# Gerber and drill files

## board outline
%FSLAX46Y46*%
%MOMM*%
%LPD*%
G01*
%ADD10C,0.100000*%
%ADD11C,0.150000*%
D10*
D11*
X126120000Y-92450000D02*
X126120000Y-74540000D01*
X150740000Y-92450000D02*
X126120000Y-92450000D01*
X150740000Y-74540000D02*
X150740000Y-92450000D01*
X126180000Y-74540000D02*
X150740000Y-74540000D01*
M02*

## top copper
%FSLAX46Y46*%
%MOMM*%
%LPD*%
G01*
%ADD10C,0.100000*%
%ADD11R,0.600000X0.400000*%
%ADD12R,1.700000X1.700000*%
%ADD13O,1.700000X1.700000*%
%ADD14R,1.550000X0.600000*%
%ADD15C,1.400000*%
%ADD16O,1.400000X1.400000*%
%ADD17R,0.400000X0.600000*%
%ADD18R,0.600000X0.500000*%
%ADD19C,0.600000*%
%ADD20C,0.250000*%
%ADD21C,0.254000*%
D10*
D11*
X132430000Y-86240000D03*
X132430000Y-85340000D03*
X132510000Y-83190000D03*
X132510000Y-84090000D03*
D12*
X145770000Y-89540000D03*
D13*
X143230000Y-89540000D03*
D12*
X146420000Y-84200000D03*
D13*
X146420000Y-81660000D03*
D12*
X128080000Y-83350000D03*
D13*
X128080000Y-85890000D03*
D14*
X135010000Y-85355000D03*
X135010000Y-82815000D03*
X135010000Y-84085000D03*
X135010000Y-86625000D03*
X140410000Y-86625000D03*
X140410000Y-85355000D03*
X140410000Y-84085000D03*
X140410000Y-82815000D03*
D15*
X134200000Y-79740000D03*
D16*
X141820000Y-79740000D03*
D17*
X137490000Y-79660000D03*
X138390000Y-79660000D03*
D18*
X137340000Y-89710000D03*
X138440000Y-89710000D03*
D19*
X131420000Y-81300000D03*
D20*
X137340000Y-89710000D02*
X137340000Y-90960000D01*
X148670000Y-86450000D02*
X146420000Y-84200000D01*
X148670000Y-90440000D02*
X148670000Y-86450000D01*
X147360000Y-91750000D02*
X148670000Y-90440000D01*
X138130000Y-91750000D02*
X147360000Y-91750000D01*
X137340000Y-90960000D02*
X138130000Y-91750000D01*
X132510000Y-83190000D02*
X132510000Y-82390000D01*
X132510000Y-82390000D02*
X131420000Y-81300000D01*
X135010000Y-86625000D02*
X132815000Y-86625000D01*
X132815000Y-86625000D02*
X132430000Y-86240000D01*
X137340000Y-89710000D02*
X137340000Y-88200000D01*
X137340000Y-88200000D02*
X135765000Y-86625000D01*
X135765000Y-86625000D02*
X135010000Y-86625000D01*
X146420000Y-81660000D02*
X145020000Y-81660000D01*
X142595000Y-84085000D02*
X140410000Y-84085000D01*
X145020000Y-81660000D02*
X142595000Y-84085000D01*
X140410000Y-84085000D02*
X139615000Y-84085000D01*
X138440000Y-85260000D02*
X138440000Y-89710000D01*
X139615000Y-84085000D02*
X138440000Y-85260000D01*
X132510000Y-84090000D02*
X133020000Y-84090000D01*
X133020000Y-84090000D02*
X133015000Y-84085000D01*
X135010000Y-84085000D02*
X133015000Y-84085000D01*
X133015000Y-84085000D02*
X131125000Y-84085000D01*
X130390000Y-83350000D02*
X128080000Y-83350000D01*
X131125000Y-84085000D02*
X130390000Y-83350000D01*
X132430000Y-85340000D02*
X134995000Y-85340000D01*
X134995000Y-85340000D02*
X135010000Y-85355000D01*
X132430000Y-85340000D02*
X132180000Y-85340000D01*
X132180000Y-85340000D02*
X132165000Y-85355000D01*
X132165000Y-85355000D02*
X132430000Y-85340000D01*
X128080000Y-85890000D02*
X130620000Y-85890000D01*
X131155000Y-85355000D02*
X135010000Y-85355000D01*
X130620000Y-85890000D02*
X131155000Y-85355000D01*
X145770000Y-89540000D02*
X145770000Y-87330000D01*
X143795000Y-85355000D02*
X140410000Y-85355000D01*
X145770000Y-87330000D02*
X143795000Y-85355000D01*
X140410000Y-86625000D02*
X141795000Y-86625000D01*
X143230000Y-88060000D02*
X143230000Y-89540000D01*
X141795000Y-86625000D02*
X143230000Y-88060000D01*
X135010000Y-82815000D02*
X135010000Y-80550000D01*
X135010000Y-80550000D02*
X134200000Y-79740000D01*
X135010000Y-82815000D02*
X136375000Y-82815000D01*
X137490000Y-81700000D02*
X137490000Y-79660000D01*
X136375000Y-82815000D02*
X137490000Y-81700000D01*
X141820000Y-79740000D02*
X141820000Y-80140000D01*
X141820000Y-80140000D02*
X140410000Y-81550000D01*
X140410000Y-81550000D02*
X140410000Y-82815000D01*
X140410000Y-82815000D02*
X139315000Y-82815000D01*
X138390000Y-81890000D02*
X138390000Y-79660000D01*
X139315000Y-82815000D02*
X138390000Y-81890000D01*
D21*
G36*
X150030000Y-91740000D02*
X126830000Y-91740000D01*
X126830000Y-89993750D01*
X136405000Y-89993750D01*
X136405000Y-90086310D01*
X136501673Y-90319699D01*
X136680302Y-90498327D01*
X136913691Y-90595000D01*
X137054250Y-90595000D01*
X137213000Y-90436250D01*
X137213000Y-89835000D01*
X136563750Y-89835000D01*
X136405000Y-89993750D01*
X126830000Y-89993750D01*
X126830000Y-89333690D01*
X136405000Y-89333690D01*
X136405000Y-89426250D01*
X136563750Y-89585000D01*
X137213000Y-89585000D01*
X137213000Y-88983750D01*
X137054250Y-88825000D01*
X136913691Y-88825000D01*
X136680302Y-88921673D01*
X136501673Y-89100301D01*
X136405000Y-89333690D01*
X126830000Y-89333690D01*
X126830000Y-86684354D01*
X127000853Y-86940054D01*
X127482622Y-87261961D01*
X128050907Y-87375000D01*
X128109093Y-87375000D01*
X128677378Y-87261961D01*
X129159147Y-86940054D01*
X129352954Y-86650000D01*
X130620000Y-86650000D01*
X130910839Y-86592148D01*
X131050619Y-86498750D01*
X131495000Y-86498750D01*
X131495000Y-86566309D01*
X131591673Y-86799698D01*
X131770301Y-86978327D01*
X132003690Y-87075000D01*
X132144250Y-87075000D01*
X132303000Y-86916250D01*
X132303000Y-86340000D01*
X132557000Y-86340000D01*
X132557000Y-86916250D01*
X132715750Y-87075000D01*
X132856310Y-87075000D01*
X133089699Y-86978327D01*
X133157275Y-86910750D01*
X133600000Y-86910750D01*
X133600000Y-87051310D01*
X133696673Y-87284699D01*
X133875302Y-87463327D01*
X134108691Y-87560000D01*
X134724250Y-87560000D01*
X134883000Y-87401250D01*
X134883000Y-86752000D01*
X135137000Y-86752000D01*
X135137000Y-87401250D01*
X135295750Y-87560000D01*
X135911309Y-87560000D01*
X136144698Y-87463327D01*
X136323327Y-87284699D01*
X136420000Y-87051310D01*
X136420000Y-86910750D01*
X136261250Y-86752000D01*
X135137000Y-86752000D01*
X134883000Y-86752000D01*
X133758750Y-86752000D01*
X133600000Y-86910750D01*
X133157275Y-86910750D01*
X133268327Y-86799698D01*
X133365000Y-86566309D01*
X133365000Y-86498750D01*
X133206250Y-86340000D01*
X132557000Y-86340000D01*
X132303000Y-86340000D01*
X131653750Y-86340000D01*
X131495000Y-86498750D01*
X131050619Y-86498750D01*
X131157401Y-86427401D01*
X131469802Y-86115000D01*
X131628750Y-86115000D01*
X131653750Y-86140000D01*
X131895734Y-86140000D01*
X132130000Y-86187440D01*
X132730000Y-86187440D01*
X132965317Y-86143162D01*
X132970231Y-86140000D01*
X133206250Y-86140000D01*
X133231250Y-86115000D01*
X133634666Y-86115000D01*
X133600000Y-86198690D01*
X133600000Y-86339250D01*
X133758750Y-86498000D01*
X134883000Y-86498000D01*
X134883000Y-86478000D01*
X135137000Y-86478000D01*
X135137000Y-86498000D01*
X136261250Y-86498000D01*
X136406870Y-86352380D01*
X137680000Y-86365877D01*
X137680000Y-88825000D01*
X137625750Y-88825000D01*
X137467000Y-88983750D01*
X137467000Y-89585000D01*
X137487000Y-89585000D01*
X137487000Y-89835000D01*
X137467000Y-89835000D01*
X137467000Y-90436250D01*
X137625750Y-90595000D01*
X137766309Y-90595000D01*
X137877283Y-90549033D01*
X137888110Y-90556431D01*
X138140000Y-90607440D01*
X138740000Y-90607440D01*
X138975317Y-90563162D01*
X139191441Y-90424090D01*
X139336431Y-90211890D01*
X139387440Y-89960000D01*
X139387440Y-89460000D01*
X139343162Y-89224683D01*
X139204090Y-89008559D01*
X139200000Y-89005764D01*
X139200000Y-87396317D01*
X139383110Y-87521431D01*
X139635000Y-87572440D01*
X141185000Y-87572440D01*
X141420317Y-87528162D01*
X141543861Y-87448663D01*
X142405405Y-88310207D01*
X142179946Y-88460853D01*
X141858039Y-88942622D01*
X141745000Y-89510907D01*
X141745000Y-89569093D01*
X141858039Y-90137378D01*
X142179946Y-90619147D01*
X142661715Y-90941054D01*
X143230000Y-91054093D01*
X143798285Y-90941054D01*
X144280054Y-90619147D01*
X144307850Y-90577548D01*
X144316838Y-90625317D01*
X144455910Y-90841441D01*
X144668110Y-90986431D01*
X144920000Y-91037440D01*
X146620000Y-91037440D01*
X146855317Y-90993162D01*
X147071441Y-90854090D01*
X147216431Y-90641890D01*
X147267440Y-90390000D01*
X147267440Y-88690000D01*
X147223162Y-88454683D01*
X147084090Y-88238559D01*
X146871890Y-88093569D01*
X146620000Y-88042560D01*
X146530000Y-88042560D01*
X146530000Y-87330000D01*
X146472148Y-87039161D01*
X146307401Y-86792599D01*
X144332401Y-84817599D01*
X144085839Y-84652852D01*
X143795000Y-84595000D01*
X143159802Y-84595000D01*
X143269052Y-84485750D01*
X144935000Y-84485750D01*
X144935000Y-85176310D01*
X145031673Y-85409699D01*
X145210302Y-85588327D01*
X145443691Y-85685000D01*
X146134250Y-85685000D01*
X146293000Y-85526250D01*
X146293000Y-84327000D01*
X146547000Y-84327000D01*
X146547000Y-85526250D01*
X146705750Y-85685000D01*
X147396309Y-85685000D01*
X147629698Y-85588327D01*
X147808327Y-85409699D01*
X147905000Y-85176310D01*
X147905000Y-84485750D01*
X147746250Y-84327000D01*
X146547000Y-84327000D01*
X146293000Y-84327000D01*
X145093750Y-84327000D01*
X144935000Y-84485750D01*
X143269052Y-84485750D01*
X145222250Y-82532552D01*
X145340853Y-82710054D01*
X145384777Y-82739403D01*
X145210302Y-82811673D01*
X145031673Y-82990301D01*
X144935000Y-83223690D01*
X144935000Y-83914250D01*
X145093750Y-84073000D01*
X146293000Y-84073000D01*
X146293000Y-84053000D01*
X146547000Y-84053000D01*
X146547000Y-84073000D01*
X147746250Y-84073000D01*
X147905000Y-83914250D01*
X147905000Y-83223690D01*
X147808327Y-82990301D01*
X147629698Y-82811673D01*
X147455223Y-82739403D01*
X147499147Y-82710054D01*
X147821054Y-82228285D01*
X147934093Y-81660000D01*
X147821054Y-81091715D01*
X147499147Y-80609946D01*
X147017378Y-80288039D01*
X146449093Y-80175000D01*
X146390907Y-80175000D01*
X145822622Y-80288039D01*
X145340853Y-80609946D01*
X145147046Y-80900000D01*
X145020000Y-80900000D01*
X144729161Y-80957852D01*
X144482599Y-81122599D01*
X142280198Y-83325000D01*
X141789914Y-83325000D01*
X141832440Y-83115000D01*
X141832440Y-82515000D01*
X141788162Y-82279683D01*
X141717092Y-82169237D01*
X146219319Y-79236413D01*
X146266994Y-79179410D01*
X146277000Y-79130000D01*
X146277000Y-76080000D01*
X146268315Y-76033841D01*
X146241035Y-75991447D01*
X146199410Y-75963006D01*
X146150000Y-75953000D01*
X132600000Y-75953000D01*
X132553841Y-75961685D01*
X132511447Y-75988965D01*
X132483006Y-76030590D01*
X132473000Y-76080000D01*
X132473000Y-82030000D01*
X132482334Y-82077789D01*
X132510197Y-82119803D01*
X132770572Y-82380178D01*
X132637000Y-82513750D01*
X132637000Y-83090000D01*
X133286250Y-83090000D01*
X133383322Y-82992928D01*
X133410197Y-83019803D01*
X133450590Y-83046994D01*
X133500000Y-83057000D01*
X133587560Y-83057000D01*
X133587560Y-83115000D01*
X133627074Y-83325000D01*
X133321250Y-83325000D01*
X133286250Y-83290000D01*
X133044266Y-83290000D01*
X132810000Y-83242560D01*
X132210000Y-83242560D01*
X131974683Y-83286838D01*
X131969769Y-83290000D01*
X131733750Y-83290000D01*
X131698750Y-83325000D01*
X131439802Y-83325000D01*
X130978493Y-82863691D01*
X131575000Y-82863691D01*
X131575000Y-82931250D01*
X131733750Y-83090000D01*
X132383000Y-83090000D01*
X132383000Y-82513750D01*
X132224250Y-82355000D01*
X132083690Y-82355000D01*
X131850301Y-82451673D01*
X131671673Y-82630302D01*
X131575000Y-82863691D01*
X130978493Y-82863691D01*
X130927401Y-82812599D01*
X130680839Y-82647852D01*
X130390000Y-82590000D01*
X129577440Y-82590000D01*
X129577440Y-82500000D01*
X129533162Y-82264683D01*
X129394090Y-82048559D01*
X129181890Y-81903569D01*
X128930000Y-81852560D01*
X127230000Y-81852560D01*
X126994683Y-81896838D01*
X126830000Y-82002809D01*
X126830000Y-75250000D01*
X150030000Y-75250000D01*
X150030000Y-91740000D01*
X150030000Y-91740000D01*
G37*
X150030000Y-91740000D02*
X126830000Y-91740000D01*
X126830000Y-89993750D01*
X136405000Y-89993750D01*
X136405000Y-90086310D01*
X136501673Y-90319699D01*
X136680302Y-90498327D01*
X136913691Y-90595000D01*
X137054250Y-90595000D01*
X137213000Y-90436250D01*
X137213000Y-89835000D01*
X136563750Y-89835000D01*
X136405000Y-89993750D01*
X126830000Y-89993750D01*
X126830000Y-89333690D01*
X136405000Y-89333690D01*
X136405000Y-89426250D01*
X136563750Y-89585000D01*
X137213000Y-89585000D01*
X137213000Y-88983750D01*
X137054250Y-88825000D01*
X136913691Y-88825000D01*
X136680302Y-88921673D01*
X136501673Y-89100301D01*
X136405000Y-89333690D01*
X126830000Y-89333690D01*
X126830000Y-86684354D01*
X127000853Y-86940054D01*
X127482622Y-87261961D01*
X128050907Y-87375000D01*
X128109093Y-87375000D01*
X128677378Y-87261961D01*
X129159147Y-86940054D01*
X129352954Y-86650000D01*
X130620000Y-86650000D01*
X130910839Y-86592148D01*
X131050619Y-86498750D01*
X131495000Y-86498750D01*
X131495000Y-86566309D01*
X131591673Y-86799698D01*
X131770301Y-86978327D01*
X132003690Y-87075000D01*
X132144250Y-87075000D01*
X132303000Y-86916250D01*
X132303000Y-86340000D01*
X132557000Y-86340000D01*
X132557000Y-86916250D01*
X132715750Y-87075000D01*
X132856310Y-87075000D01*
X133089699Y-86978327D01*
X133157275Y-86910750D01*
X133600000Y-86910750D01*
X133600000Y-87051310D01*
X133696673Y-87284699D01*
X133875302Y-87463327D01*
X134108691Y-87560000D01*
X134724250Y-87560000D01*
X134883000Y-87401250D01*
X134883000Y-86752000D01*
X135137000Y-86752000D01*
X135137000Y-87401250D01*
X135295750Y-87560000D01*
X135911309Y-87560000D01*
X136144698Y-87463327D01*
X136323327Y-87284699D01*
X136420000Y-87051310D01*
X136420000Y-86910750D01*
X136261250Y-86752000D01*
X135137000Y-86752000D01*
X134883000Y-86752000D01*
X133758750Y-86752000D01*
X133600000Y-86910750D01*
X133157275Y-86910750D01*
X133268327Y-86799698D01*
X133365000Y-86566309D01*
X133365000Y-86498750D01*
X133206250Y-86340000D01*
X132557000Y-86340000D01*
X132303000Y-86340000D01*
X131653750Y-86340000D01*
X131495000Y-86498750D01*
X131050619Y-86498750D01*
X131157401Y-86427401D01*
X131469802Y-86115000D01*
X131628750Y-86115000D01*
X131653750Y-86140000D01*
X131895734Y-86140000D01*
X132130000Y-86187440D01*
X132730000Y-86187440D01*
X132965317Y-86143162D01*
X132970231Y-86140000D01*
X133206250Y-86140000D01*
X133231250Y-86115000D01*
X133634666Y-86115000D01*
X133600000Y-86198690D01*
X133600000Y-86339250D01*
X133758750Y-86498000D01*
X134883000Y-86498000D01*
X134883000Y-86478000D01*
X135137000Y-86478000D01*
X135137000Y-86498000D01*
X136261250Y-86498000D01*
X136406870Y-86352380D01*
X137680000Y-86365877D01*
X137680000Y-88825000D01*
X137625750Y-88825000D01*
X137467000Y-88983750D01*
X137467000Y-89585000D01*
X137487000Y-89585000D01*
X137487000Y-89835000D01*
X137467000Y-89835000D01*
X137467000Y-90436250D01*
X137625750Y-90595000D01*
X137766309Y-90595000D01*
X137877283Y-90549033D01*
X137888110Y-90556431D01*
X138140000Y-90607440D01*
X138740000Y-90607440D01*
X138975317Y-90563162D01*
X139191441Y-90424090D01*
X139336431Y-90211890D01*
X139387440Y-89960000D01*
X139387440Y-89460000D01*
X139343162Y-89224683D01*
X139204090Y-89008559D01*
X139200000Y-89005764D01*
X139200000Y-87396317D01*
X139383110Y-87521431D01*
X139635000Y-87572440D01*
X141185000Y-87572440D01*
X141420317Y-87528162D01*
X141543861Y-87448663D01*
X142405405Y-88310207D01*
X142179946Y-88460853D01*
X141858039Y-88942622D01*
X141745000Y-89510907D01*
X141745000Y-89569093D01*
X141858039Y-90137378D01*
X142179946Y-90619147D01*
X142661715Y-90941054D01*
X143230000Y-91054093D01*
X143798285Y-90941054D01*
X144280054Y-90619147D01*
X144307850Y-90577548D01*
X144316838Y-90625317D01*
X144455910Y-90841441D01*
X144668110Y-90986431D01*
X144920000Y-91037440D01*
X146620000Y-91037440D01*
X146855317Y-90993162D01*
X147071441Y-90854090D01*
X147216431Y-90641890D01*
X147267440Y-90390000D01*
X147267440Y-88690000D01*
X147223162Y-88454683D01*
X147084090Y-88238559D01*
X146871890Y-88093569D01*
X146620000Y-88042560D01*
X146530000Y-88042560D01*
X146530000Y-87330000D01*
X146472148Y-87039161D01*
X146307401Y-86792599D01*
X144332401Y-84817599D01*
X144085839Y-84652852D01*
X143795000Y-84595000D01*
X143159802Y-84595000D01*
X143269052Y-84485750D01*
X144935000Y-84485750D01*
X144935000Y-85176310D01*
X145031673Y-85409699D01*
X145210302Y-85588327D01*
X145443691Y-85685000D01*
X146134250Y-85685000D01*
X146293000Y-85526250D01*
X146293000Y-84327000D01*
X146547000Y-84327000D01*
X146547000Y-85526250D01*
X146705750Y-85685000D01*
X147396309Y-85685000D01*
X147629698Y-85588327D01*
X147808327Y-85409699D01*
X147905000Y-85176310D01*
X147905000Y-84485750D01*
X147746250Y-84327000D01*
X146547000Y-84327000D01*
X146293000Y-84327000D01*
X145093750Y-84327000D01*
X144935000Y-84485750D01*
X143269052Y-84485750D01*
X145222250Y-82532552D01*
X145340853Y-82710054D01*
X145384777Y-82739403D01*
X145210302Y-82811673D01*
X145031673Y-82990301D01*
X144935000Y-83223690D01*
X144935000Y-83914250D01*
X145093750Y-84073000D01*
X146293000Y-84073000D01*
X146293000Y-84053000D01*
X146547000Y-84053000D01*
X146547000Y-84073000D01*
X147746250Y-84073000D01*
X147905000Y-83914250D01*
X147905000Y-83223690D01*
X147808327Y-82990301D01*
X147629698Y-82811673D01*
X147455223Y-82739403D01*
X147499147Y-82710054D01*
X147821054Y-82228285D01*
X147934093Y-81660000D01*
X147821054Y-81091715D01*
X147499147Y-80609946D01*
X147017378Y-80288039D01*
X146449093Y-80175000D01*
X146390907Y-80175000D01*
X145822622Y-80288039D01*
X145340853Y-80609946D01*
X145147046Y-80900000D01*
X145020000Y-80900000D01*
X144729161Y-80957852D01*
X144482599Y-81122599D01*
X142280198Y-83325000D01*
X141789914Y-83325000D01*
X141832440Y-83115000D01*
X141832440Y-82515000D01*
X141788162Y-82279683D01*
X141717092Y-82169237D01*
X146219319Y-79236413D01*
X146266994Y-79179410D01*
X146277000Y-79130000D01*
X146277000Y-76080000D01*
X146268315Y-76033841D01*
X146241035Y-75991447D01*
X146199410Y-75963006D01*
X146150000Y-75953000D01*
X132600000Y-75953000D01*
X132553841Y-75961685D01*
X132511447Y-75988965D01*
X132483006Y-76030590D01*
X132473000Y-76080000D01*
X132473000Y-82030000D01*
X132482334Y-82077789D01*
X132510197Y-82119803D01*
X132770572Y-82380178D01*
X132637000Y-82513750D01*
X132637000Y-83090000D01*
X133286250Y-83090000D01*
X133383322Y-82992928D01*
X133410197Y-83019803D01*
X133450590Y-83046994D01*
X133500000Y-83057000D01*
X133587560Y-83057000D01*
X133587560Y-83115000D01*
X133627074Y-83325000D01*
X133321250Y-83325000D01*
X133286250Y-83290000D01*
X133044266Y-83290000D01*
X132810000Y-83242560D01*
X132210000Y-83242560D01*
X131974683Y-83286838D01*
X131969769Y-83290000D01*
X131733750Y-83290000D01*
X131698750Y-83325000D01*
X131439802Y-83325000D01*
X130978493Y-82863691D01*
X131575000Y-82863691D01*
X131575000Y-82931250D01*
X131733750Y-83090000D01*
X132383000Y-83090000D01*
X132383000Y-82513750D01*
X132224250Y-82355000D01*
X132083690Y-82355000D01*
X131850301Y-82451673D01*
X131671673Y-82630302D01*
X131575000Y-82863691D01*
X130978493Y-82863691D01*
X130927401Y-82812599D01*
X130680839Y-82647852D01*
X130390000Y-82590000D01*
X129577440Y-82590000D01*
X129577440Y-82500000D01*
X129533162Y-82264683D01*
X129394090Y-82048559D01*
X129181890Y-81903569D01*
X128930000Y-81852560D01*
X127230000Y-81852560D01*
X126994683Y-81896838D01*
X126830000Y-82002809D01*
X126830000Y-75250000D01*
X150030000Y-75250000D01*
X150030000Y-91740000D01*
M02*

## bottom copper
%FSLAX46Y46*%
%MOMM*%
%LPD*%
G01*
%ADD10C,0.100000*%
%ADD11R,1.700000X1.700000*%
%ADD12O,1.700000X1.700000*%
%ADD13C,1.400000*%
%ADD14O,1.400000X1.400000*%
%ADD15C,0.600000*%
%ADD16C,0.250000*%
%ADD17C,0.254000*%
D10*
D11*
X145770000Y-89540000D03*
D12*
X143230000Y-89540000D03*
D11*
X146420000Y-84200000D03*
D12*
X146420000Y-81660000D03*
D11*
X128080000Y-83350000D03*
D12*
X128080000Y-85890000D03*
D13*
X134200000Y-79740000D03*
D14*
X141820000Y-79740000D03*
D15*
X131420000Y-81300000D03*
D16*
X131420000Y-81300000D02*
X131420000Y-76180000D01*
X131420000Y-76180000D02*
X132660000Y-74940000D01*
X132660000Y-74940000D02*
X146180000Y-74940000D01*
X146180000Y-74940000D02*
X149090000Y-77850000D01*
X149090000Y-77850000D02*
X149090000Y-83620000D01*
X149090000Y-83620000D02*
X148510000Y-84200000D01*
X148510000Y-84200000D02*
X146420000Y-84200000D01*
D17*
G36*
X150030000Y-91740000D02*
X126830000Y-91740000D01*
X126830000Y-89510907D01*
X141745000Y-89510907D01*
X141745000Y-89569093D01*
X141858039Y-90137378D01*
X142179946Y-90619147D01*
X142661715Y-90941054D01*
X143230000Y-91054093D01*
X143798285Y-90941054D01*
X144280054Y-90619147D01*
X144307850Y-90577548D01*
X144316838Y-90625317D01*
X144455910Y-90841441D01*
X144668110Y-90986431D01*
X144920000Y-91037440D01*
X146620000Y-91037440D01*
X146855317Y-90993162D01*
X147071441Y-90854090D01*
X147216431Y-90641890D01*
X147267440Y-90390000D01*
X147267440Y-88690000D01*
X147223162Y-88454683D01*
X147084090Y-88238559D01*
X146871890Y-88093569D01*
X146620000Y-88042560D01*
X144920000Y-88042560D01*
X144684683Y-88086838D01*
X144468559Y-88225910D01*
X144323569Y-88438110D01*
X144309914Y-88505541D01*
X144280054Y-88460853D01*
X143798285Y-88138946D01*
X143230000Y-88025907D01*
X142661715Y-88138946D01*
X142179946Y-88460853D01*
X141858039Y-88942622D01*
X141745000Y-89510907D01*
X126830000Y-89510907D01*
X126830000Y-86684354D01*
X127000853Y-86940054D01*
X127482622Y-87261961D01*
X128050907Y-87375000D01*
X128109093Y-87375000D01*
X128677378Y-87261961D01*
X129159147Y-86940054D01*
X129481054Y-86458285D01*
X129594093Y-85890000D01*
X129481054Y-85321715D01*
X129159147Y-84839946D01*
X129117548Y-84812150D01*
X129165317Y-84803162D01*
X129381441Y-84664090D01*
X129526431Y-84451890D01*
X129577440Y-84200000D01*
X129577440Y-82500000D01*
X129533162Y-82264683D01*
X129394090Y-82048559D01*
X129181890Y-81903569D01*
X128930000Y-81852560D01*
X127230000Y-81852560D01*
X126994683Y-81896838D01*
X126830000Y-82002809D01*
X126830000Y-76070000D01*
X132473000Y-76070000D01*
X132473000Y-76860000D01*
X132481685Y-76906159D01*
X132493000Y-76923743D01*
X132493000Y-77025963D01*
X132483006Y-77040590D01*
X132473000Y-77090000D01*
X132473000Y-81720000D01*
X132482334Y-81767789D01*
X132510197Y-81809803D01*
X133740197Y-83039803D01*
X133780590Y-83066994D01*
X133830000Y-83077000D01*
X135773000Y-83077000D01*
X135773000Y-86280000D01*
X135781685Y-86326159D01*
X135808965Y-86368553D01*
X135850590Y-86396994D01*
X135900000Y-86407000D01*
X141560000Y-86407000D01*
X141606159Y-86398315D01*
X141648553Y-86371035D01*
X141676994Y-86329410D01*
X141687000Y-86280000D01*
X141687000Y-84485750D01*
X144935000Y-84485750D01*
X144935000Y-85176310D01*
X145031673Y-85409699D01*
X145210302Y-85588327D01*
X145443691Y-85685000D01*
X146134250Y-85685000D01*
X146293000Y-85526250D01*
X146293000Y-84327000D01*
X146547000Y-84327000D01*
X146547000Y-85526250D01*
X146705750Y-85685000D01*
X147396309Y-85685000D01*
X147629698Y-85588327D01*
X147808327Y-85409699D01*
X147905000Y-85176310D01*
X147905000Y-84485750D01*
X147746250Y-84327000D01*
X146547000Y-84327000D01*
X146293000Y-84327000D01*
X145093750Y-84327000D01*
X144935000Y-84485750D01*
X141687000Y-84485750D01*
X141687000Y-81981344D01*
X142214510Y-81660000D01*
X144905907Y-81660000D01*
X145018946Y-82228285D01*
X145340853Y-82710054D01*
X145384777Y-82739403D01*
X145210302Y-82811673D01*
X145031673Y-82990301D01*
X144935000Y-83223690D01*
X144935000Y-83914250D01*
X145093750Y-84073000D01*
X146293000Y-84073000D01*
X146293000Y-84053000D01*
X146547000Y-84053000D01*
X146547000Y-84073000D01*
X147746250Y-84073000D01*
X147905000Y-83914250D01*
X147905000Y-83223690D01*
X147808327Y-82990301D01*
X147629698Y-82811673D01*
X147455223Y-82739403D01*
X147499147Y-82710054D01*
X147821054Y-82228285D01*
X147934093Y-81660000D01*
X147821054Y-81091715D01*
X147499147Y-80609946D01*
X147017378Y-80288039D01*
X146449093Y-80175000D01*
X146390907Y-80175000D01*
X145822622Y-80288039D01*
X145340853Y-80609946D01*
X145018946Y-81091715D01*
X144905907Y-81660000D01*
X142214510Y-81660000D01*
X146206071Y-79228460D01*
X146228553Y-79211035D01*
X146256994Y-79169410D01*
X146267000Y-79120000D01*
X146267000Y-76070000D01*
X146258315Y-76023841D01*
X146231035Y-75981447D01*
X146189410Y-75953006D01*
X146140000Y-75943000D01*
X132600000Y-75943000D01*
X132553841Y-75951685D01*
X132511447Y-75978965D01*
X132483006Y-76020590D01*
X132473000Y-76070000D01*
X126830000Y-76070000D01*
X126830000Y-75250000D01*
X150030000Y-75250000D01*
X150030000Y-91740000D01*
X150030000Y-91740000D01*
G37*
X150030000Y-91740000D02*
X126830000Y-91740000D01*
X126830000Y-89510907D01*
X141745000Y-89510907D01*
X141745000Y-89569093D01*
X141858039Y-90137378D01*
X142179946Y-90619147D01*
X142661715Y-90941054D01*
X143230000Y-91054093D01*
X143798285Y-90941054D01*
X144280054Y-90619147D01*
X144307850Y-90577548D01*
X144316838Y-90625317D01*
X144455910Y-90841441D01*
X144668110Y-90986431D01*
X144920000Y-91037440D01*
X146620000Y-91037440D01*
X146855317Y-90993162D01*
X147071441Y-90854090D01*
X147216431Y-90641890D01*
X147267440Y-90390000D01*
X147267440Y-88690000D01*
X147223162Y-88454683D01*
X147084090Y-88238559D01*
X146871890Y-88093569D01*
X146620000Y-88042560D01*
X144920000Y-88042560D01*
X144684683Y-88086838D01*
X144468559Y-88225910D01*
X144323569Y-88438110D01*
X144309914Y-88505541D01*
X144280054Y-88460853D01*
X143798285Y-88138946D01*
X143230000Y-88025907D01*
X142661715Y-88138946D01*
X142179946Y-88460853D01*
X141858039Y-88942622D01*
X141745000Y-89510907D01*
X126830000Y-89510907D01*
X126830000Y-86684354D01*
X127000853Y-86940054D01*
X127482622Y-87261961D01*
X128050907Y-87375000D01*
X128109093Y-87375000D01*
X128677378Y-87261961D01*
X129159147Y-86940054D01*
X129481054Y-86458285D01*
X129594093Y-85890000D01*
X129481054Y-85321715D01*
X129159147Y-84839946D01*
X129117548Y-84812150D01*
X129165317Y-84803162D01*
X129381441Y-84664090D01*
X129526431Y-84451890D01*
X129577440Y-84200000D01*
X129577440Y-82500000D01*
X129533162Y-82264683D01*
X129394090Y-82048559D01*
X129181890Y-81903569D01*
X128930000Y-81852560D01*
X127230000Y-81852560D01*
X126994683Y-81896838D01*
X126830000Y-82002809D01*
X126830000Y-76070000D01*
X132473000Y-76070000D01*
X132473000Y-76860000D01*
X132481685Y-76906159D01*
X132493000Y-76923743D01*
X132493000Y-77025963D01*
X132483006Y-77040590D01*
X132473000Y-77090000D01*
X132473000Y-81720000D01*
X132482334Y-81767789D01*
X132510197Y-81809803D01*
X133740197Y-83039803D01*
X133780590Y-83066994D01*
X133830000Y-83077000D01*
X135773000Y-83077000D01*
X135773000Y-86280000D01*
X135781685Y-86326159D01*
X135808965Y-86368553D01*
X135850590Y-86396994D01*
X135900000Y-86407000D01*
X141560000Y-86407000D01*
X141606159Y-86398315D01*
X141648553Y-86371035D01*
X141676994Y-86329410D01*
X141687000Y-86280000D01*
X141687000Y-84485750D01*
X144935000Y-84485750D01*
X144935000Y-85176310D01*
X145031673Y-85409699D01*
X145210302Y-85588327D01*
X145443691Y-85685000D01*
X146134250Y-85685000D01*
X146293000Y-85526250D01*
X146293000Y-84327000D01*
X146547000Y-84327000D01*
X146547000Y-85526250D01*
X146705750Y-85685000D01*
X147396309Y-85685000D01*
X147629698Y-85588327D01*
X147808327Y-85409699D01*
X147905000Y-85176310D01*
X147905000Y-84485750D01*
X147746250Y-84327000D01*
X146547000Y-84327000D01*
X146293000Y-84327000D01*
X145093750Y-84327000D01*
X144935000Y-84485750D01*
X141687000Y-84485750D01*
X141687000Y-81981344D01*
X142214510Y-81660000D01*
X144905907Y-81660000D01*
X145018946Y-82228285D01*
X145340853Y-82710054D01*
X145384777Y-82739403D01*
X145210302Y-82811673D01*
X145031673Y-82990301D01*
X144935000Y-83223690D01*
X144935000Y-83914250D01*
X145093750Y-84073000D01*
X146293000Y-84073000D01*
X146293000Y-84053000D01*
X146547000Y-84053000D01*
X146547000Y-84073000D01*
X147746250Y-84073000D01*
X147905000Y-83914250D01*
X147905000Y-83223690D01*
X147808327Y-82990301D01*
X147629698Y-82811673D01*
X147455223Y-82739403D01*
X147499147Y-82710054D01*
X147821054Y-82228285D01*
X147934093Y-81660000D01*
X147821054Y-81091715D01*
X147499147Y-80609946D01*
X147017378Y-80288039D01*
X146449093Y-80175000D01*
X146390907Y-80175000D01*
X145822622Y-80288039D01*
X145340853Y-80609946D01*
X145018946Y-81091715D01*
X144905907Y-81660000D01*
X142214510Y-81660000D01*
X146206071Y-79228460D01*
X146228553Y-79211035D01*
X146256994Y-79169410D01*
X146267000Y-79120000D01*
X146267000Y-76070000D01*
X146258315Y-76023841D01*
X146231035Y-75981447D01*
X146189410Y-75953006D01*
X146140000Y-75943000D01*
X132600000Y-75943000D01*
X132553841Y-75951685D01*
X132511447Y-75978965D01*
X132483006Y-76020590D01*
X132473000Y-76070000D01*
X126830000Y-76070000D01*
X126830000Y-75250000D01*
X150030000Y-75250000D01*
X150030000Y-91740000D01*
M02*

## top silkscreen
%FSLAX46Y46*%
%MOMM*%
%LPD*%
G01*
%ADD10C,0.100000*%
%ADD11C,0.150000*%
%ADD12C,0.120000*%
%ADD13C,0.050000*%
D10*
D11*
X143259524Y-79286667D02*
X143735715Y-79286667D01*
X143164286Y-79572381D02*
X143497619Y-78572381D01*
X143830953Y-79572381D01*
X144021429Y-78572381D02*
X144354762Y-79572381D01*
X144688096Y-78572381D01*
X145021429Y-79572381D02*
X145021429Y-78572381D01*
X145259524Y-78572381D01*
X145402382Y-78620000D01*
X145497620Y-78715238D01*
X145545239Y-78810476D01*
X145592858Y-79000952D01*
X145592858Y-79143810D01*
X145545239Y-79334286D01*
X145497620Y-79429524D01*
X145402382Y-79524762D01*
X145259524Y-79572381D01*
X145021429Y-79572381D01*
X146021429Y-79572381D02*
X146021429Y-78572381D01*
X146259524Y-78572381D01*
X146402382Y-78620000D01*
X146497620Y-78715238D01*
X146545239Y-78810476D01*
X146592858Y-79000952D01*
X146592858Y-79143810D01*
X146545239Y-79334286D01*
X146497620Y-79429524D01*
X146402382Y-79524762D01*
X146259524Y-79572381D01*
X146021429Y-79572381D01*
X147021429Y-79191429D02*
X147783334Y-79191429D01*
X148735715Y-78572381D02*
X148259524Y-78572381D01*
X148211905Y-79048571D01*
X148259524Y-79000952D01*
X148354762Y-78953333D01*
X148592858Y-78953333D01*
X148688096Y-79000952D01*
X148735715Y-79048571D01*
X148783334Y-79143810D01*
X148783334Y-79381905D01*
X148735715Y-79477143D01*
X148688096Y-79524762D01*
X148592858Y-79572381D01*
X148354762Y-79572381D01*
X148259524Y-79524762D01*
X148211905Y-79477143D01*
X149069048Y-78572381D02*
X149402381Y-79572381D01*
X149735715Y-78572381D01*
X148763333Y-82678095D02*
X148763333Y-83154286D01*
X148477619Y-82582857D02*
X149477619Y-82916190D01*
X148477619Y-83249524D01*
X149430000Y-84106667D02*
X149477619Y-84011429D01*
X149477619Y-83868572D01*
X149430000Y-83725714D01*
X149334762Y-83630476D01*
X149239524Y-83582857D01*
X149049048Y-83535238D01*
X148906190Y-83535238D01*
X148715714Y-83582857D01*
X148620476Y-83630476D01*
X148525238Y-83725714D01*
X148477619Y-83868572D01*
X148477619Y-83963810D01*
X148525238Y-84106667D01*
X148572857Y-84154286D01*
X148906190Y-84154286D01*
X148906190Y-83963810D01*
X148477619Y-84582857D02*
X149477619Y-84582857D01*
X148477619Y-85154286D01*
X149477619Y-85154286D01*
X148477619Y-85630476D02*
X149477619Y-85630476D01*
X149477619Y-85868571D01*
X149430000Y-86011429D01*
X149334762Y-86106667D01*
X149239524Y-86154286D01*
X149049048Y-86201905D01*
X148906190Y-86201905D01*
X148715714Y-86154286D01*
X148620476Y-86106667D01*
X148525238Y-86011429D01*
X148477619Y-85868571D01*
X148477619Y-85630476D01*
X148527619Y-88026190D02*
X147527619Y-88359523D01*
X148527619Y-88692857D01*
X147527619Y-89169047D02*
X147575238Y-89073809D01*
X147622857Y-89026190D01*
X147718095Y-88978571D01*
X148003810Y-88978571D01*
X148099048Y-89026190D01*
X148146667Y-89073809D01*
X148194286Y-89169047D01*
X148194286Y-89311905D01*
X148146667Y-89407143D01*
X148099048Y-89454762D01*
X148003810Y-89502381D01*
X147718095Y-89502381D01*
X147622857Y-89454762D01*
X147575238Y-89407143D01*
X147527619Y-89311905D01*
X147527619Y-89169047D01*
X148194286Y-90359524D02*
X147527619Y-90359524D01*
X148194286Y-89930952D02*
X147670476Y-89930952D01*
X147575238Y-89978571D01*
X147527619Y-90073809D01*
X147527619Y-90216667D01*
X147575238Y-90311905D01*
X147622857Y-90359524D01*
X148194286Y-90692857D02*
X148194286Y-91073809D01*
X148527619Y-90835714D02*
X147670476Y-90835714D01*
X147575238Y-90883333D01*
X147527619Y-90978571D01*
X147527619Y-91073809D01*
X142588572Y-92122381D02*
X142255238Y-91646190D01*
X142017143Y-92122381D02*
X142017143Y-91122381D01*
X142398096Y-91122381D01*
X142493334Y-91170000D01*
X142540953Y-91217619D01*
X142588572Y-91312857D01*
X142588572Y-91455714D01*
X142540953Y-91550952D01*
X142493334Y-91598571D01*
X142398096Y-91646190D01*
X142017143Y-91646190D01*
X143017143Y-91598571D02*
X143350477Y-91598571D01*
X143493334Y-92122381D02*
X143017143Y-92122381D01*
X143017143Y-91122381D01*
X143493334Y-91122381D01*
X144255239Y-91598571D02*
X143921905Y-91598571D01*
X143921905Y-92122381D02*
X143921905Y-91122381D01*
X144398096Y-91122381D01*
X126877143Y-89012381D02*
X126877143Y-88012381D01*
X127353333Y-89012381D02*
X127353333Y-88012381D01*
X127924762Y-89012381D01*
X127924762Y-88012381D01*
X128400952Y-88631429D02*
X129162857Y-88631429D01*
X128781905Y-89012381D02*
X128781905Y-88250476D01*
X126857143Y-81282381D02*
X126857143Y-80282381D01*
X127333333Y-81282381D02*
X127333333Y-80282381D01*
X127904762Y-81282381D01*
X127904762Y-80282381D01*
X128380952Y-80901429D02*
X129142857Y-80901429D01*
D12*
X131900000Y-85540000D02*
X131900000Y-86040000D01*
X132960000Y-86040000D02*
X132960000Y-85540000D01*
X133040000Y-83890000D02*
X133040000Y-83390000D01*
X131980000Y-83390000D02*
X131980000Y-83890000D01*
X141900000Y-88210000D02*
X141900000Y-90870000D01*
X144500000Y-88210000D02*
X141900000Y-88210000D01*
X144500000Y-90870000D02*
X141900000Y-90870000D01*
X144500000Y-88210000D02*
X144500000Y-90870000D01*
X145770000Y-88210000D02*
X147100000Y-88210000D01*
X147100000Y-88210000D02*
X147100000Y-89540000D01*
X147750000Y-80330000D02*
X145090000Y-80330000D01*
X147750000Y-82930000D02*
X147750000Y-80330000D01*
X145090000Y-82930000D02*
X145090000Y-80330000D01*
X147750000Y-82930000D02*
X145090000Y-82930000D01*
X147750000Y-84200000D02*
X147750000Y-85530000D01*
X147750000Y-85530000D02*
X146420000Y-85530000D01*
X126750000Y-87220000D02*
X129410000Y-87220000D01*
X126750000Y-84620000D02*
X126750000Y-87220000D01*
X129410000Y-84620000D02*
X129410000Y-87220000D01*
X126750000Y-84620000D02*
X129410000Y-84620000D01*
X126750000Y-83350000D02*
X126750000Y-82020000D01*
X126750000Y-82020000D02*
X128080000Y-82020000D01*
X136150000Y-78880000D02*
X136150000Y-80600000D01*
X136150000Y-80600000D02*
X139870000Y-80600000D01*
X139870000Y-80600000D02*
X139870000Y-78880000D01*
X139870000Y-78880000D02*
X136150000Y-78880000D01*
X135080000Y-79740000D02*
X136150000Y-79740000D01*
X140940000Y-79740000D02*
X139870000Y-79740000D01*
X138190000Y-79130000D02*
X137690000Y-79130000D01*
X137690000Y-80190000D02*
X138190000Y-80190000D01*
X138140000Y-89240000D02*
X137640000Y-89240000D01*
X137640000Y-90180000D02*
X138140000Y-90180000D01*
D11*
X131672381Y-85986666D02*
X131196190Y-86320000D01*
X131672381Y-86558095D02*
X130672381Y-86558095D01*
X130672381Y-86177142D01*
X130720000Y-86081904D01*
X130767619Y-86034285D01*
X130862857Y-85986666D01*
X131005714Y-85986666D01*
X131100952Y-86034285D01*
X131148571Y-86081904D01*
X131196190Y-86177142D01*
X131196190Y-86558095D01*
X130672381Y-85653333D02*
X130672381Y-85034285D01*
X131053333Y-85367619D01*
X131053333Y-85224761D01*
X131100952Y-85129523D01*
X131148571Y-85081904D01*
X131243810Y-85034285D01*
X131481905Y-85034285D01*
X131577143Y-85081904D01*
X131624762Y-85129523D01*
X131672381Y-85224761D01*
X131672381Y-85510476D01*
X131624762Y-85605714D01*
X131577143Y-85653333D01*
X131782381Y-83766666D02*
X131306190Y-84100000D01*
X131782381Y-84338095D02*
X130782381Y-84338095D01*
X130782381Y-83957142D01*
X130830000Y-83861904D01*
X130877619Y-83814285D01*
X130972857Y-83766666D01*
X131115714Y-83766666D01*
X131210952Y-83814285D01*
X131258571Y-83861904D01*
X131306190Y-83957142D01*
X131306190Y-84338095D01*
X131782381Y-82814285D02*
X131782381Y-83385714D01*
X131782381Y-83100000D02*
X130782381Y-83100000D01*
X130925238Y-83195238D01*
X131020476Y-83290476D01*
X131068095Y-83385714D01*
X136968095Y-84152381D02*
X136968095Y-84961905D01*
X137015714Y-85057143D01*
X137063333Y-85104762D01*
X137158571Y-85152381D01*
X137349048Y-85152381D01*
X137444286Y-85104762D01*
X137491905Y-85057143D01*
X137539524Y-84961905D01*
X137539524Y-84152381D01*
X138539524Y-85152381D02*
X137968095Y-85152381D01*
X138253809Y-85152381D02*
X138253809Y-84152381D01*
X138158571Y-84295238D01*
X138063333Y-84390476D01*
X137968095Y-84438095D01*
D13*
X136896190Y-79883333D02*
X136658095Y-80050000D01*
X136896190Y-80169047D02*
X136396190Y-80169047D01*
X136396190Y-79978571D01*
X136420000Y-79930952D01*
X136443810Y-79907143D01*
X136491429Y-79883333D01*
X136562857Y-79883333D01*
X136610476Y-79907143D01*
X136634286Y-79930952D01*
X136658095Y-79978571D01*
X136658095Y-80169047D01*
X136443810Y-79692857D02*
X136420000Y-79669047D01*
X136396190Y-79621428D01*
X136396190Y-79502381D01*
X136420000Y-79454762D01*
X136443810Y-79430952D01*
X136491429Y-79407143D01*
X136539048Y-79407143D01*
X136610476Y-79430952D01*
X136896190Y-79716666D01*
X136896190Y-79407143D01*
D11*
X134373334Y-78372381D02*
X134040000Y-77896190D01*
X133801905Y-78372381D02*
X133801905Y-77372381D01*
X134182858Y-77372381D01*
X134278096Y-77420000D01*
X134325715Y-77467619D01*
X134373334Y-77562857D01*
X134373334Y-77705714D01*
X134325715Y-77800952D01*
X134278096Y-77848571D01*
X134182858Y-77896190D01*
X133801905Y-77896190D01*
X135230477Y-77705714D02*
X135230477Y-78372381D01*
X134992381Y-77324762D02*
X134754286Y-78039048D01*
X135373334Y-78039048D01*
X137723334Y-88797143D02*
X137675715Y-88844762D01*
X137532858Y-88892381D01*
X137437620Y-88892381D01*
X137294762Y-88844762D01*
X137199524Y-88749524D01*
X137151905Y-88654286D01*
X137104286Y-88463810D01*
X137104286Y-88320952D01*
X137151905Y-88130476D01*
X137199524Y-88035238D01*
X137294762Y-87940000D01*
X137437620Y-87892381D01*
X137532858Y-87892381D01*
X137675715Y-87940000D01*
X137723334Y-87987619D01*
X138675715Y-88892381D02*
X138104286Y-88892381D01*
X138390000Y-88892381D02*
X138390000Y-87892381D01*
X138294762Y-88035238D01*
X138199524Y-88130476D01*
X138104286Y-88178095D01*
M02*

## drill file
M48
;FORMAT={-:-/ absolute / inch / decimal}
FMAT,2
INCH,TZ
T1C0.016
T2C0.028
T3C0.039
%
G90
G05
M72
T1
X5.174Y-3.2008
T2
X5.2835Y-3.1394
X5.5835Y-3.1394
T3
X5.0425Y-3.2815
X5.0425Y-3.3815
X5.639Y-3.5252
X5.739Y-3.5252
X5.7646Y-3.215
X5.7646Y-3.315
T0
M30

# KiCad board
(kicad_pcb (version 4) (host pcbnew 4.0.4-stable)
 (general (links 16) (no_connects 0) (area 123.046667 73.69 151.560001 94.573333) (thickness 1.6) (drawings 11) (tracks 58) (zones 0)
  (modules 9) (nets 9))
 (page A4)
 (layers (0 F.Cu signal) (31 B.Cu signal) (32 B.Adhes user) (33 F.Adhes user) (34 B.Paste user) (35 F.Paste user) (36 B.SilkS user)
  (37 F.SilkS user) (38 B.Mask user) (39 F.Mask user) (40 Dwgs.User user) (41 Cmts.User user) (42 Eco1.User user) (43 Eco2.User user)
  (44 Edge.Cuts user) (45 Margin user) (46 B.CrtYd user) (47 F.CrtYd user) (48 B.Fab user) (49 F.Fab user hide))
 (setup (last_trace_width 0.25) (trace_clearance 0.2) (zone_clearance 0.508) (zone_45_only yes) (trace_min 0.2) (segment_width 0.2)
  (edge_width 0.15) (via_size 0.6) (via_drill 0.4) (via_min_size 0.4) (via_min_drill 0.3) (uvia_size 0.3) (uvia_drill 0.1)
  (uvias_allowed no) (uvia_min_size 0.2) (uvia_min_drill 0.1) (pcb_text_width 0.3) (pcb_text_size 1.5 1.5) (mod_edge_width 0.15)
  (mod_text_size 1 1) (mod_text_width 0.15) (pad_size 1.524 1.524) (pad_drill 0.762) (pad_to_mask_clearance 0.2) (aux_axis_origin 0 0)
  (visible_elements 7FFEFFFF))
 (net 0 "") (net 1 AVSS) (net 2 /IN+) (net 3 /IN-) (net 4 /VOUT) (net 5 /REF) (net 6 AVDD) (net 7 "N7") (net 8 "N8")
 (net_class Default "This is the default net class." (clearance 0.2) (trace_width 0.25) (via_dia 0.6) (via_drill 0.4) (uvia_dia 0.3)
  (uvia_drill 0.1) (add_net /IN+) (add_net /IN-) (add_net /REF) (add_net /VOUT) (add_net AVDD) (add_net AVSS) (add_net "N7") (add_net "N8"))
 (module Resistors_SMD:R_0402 (layer F.Cu) (at 132.43 85.79 90)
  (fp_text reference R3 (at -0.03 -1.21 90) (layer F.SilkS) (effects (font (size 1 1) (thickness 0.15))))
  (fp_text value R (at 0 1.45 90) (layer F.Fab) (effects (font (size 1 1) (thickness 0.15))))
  (fp_line (start 0.25 -0.53) (end -0.25 -0.53) (layer F.SilkS) (width 0.12))
  (fp_line (start -0.25 0.53) (end 0.25 0.53) (layer F.SilkS) (width 0.12))
  (pad 1 smd rect (at -0.45 0 90) (size 0.4 0.6) (layers F.Cu F.Paste F.Mask) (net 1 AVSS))
  (pad 2 smd rect (at 0.45 0 90) (size 0.4 0.6) (layers F.Cu F.Paste F.Mask) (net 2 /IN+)))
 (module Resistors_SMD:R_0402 (layer F.Cu) (at 132.51 83.64 270)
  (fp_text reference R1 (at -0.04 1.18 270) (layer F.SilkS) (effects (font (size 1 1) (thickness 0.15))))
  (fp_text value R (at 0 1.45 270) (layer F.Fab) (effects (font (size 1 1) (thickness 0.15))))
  (fp_line (start 0.25 -0.53) (end -0.25 -0.53) (layer F.SilkS) (width 0.12))
  (fp_line (start -0.25 0.53) (end 0.25 0.53) (layer F.SilkS) (width 0.12))
  (pad 1 smd rect (at -0.45 0 270) (size 0.4 0.6) (layers F.Cu F.Paste F.Mask) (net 1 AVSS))
  (pad 2 smd rect (at 0.45 0 270) (size 0.4 0.6) (layers F.Cu F.Paste F.Mask) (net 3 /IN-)))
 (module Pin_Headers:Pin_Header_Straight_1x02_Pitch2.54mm (layer F.Cu) (at 145.77 89.54 270)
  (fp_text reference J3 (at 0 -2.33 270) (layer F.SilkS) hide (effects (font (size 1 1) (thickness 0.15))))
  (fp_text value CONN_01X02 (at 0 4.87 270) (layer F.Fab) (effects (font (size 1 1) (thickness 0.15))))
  (fp_line (start -1.33 3.87) (end 1.33 3.87) (layer F.SilkS) (width 0.12))
  (fp_line (start -1.33 1.27) (end -1.33 3.87) (layer F.SilkS) (width 0.12))
  (fp_line (start 1.33 1.27) (end 1.33 3.87) (layer F.SilkS) (width 0.12))
  (fp_line (start -1.33 1.27) (end 1.33 1.27) (layer F.SilkS) (width 0.12))
  (fp_line (start -1.33 0) (end -1.33 -1.33) (layer F.SilkS) (width 0.12))
  (fp_line (start -1.33 -1.33) (end 0 -1.33) (layer F.SilkS) (width 0.12))
  (pad 1 thru_hole rect (at 0 0 270) (size 1.7 1.7) (drill 1) (layers *.Cu *.Mask) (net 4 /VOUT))
  (pad 2 thru_hole oval (at 0 2.54 270) (size 1.7 1.7) (drill 1) (layers *.Cu *.Mask) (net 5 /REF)))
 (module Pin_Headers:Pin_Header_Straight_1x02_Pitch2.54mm (layer F.Cu) (at 146.42 84.2 180)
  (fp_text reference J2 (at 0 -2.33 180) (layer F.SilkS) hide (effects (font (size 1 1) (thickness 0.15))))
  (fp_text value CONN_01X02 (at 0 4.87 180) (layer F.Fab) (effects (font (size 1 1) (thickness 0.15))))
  (fp_line (start -1.33 3.87) (end 1.33 3.87) (layer F.SilkS) (width 0.12))
  (fp_line (start -1.33 1.27) (end -1.33 3.87) (layer F.SilkS) (width 0.12))
  (fp_line (start 1.33 1.27) (end 1.33 3.87) (layer F.SilkS) (width 0.12))
  (fp_line (start -1.33 1.27) (end 1.33 1.27) (layer F.SilkS) (width 0.12))
  (fp_line (start -1.33 0) (end -1.33 -1.33) (layer F.SilkS) (width 0.12))
  (fp_line (start -1.33 -1.33) (end 0 -1.33) (layer F.SilkS) (width 0.12))
  (pad 1 thru_hole rect (at 0 0 180) (size 1.7 1.7) (drill 1) (layers *.Cu *.Mask) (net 1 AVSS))
  (pad 2 thru_hole oval (at 0 2.54 180) (size 1.7 1.7) (drill 1) (layers *.Cu *.Mask) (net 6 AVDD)))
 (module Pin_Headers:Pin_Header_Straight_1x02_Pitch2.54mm (layer F.Cu) (at 128.08 83.35)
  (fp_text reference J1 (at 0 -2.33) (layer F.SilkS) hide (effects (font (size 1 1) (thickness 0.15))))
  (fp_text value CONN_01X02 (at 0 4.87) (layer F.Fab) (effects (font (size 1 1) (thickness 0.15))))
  (fp_line (start -1.33 3.87) (end 1.33 3.87) (layer F.SilkS) (width 0.12))
  (fp_line (start -1.33 1.27) (end -1.33 3.87) (layer F.SilkS) (width 0.12))
  (fp_line (start 1.33 1.27) (end 1.33 3.87) (layer F.SilkS) (width 0.12))
  (fp_line (start -1.33 1.27) (end 1.33 1.27) (layer F.SilkS) (width 0.12))
  (fp_line (start -1.33 0) (end -1.33 -1.33) (layer F.SilkS) (width 0.12))
  (fp_line (start -1.33 -1.33) (end 0 -1.33) (layer F.SilkS) (width 0.12))
  (pad 1 thru_hole rect (at 0 0) (size 1.7 1.7) (drill 1) (layers *.Cu *.Mask) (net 3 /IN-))
  (pad 2 thru_hole oval (at 0 2.54) (size 1.7 1.7) (drill 1) (layers *.Cu *.Mask) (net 2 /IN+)))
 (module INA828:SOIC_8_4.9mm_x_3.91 (layer F.Cu) (at 137.71 84.72)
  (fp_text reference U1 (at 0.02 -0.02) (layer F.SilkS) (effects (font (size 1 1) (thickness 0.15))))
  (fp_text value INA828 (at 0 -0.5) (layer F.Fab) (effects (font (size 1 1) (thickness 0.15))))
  (pad 3 smd rect (at -2.7 0.635) (size 1.55 0.6) (layers F.Cu F.Paste F.Mask) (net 2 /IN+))
  (pad 1 smd rect (at -2.7 -1.905) (size 1.55 0.6) (layers F.Cu F.Paste F.Mask) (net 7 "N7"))
  (pad 2 smd rect (at -2.7 -0.635) (size 1.55 0.6) (layers F.Cu F.Paste F.Mask) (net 3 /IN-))
  (pad 4 smd rect (at -2.7 1.905) (size 1.55 0.6) (layers F.Cu F.Paste F.Mask) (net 1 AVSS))
  (pad 5 smd rect (at 2.7 1.905) (size 1.55 0.6) (layers F.Cu F.Paste F.Mask) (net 5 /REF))
  (pad 6 smd rect (at 2.7 0.635) (size 1.55 0.6) (layers F.Cu F.Paste F.Mask) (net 4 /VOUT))
  (pad 7 smd rect (at 2.7 -0.635) (size 1.55 0.6) (layers F.Cu F.Paste F.Mask) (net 6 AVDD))
  (pad 8 smd rect (at 2.7 -1.905) (size 1.55 0.6) (layers F.Cu F.Paste F.Mask) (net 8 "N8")))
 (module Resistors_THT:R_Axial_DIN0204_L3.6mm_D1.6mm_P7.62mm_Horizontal (layer F.Cu) (at 134.2 79.74)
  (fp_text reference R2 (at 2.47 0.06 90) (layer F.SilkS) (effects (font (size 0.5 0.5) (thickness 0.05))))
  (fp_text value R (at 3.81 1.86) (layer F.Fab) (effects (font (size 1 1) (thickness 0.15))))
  (fp_line (start 1.95 -0.86) (end 1.95 0.86) (layer F.SilkS) (width 0.12))
  (fp_line (start 1.95 0.86) (end 5.67 0.86) (layer F.SilkS) (width 0.12))
  (fp_line (start 5.67 0.86) (end 5.67 -0.86) (layer F.SilkS) (width 0.12))
  (fp_line (start 5.67 -0.86) (end 1.95 -0.86) (layer F.SilkS) (width 0.12))
  (fp_line (start 0.88 0) (end 1.95 0) (layer F.SilkS) (width 0.12))
  (fp_line (start 6.74 0) (end 5.67 0) (layer F.SilkS) (width 0.12))
  (pad 1 thru_hole circle (at 0 0) (size 1.4 1.4) (drill 0.7) (layers *.Cu *.Mask) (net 7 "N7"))
  (pad 2 thru_hole oval (at 7.62 0) (size 1.4 1.4) (drill 0.7) (layers *.Cu *.Mask) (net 8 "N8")))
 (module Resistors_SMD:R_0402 (layer F.Cu) (at 137.94 79.66)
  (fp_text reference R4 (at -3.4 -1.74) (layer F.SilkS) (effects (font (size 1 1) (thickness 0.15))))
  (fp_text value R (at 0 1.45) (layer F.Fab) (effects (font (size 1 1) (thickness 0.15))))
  (fp_line (start 0.25 -0.53) (end -0.25 -0.53) (layer F.SilkS) (width 0.12))
  (fp_line (start -0.25 0.53) (end 0.25 0.53) (layer F.SilkS) (width 0.12))
  (pad 1 smd rect (at -0.45 0) (size 0.4 0.6) (layers F.Cu F.Paste F.Mask) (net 7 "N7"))
  (pad 2 smd rect (at 0.45 0) (size 0.4 0.6) (layers F.Cu F.Paste F.Mask) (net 8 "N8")))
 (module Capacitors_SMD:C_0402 (layer F.Cu) (at 137.89 89.71)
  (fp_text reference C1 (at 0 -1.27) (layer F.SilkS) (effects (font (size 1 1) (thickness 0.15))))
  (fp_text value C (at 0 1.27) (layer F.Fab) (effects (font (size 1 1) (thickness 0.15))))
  (fp_line (start 0.25 -0.47) (end -0.25 -0.47) (layer F.SilkS) (width 0.12))
  (fp_line (start -0.25 0.47) (end 0.25 0.47) (layer F.SilkS) (width 0.12))
  (pad 1 smd rect (at -0.55 0) (size 0.6 0.5) (layers F.Cu F.Paste F.Mask) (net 1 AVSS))
  (pad 2 smd rect (at 0.55 0) (size 0.6 0.5) (layers F.Cu F.Paste F.Mask) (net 6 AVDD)))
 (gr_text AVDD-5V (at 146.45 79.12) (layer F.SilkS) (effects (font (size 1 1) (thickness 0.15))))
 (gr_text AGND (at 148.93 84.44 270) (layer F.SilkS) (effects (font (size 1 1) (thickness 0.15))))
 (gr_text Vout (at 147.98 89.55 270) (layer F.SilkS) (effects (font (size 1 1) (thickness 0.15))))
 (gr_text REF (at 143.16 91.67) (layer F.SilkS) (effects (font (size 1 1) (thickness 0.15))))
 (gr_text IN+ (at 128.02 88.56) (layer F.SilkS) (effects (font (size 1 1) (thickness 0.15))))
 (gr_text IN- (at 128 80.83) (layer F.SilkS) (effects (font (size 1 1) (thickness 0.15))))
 (gr_line (start 126.12 92.45) (end 126.12 74.54) (angle 90) (layer Edge.Cuts) (width 0.15))
 (gr_line (start 150.74 92.45) (end 126.12 92.45) (angle 90) (layer Edge.Cuts) (width 0.15))
 (gr_line (start 150.74 74.54) (end 150.74 92.45) (angle 90) (layer Edge.Cuts) (width 0.15))
 (gr_line (start 126.18 74.54) (end 150.74 74.54) (angle 90) (layer Edge.Cuts) (width 0.15))
 (segment (start 137.34 89.71) (end 137.34 90.96) (width 0.25) (layer F.Cu) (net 1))
 (segment (start 148.67 86.45) (end 146.42 84.2) (width 0.25) (layer F.Cu) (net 1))
 (segment (start 148.67 90.44) (end 148.67 86.45) (width 0.25) (layer F.Cu) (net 1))
 (segment (start 147.36 91.75) (end 148.67 90.44) (width 0.25) (layer F.Cu) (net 1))
 (segment (start 138.13 91.75) (end 147.36 91.75) (width 0.25) (layer F.Cu) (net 1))
 (segment (start 137.34 90.96) (end 138.13 91.75) (width 0.25) (layer F.Cu) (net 1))
 (segment (start 131.42 81.3) (end 131.42 76.18) (width 0.25) (layer B.Cu) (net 1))
 (segment (start 131.42 76.18) (end 132.66 74.94) (width 0.25) (layer B.Cu) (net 1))
 (segment (start 132.66 74.94) (end 146.18 74.94) (width 0.25) (layer B.Cu) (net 1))
 (segment (start 146.18 74.94) (end 149.09 77.85) (width 0.25) (layer B.Cu) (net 1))
 (segment (start 149.09 77.85) (end 149.09 83.62) (width 0.25) (layer B.Cu) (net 1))
 (segment (start 149.09 83.62) (end 148.51 84.2) (width 0.25) (layer B.Cu) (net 1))
 (segment (start 148.51 84.2) (end 146.42 84.2) (width 0.25) (layer B.Cu) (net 1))
 (segment (start 132.51 83.19) (end 132.51 82.39) (width 0.25) (layer F.Cu) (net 1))
 (via (at 131.42 81.3) (size 0.6) (drill 0.4) (layers F.Cu B.Cu) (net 1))
 (segment (start 132.51 82.39) (end 131.42 81.3) (width 0.25) (layer F.Cu) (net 1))
 (segment (start 135.01 86.625) (end 132.815 86.625) (width 0.25) (layer F.Cu) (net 1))
 (segment (start 132.815 86.625) (end 132.43 86.24) (width 0.25) (layer F.Cu) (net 1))
 (segment (start 137.34 89.71) (end 137.34 88.2) (width 0.25) (layer F.Cu) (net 1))
 (segment (start 137.34 88.2) (end 135.765 86.625) (width 0.25) (layer F.Cu) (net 1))
 (segment (start 135.765 86.625) (end 135.01 86.625) (width 0.25) (layer F.Cu) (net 1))
 (segment (start 146.42 81.66) (end 145.02 81.66) (width 0.25) (layer F.Cu) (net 6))
 (segment (start 142.595 84.085) (end 140.41 84.085) (width 0.25) (layer F.Cu) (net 6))
 (segment (start 145.02 81.66) (end 142.595 84.085) (width 0.25) (layer F.Cu) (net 6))
 (segment (start 140.41 84.085) (end 139.615 84.085) (width 0.25) (layer F.Cu) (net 6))
 (segment (start 138.44 85.26) (end 138.44 89.71) (width 0.25) (layer F.Cu) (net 6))
 (segment (start 139.615 84.085) (end 138.44 85.26) (width 0.25) (layer F.Cu) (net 6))
 (segment (start 132.51 84.09) (end 133.02 84.09) (width 0.25) (layer F.Cu) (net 3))
 (segment (start 133.02 84.09) (end 133.015 84.085) (width 0.25) (layer F.Cu) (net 3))
 (segment (start 135.01 84.085) (end 133.015 84.085) (width 0.25) (layer F.Cu) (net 3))
 (segment (start 133.015 84.085) (end 131.125 84.085) (width 0.25) (layer F.Cu) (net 3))
 (segment (start 130.39 83.35) (end 128.08 83.35) (width 0.25) (layer F.Cu) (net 3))
 (segment (start 131.125 84.085) (end 130.39 83.35) (width 0.25) (layer F.Cu) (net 3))
 (segment (start 132.43 85.34) (end 134.995 85.34) (width 0.25) (layer F.Cu) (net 2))
 (segment (start 134.995 85.34) (end 135.01 85.355) (width 0.25) (layer F.Cu) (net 2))
 (segment (start 132.43 85.34) (end 132.18 85.34) (width 0.25) (layer F.Cu) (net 2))
 (segment (start 132.18 85.34) (end 132.165 85.355) (width 0.25) (layer F.Cu) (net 2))
 (segment (start 132.165 85.355) (end 132.43 85.34) (width 0.25) (layer F.Cu) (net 2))
 (segment (start 128.08 85.89) (end 130.62 85.89) (width 0.25) (layer F.Cu) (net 2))
 (segment (start 131.155 85.355) (end 135.01 85.355) (width 0.25) (layer F.Cu) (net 2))
 (segment (start 130.62 85.89) (end 131.155 85.355) (width 0.25) (layer F.Cu) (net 2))
 (segment (start 145.77 89.54) (end 145.77 87.33) (width 0.25) (layer F.Cu) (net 4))
 (segment (start 143.795 85.355) (end 140.41 85.355) (width 0.25) (layer F.Cu) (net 4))
 (segment (start 145.77 87.33) (end 143.795 85.355) (width 0.25) (layer F.Cu) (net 4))
 (segment (start 140.41 86.625) (end 141.795 86.625) (width 0.25) (layer F.Cu) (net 5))
 (segment (start 143.23 88.06) (end 143.23 89.54) (width 0.25) (layer F.Cu) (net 5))
 (segment (start 141.795 86.625) (end 143.23 88.06) (width 0.25) (layer F.Cu) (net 5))
 (segment (start 135.01 82.815) (end 135.01 80.55) (width 0.25) (layer F.Cu) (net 7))
 (segment (start 135.01 80.55) (end 134.2 79.74) (width 0.25) (layer F.Cu) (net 7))
 (segment (start 135.01 82.815) (end 136.375 82.815) (width 0.25) (layer F.Cu) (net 7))
 (segment (start 137.49 81.7) (end 137.49 79.66) (width 0.25) (layer F.Cu) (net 7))
 (segment (start 136.375 82.815) (end 137.49 81.7) (width 0.25) (layer F.Cu) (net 7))
 (segment (start 141.82 79.74) (end 141.82 80.14) (width 0.25) (layer F.Cu) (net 8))
 (segment (start 141.82 80.14) (end 140.41 81.55) (width 0.25) (layer F.Cu) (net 8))
 (segment (start 140.41 81.55) (end 140.41 82.815) (width 0.25) (layer F.Cu) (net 8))
 (segment (start 140.41 82.815) (end 139.315 82.815) (width 0.25) (layer F.Cu) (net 8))
 (segment (start 138.39 81.89) (end 138.39 79.66) (width 0.25) (layer F.Cu) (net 8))
 (segment (start 139.315 82.815) (end 138.39 81.89) (width 0.25) (layer F.Cu) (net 8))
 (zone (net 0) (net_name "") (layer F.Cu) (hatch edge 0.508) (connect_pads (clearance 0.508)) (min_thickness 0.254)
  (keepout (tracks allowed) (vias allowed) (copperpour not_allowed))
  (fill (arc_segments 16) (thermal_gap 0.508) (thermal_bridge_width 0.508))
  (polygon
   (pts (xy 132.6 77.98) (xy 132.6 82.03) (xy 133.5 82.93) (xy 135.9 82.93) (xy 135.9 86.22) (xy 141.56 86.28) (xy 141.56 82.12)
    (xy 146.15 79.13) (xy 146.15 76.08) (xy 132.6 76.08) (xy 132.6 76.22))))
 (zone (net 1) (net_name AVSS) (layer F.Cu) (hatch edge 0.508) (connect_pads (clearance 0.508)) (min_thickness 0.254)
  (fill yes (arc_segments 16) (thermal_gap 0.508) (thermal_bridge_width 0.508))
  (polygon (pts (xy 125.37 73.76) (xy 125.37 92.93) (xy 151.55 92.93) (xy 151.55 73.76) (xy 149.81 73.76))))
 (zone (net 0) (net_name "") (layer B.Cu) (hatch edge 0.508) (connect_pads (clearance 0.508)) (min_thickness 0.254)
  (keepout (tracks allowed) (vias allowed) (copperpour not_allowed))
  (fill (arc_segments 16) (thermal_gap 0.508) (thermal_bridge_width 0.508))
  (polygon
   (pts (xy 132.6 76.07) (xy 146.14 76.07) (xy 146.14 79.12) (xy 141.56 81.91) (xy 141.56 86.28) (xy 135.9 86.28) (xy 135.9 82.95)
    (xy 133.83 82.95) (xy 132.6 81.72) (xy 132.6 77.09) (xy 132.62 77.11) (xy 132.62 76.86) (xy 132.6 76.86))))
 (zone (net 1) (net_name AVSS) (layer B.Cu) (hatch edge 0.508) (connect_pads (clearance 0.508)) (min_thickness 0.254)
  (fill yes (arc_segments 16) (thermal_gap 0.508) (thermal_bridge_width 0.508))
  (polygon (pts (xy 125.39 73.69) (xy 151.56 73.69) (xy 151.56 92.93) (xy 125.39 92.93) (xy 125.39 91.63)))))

